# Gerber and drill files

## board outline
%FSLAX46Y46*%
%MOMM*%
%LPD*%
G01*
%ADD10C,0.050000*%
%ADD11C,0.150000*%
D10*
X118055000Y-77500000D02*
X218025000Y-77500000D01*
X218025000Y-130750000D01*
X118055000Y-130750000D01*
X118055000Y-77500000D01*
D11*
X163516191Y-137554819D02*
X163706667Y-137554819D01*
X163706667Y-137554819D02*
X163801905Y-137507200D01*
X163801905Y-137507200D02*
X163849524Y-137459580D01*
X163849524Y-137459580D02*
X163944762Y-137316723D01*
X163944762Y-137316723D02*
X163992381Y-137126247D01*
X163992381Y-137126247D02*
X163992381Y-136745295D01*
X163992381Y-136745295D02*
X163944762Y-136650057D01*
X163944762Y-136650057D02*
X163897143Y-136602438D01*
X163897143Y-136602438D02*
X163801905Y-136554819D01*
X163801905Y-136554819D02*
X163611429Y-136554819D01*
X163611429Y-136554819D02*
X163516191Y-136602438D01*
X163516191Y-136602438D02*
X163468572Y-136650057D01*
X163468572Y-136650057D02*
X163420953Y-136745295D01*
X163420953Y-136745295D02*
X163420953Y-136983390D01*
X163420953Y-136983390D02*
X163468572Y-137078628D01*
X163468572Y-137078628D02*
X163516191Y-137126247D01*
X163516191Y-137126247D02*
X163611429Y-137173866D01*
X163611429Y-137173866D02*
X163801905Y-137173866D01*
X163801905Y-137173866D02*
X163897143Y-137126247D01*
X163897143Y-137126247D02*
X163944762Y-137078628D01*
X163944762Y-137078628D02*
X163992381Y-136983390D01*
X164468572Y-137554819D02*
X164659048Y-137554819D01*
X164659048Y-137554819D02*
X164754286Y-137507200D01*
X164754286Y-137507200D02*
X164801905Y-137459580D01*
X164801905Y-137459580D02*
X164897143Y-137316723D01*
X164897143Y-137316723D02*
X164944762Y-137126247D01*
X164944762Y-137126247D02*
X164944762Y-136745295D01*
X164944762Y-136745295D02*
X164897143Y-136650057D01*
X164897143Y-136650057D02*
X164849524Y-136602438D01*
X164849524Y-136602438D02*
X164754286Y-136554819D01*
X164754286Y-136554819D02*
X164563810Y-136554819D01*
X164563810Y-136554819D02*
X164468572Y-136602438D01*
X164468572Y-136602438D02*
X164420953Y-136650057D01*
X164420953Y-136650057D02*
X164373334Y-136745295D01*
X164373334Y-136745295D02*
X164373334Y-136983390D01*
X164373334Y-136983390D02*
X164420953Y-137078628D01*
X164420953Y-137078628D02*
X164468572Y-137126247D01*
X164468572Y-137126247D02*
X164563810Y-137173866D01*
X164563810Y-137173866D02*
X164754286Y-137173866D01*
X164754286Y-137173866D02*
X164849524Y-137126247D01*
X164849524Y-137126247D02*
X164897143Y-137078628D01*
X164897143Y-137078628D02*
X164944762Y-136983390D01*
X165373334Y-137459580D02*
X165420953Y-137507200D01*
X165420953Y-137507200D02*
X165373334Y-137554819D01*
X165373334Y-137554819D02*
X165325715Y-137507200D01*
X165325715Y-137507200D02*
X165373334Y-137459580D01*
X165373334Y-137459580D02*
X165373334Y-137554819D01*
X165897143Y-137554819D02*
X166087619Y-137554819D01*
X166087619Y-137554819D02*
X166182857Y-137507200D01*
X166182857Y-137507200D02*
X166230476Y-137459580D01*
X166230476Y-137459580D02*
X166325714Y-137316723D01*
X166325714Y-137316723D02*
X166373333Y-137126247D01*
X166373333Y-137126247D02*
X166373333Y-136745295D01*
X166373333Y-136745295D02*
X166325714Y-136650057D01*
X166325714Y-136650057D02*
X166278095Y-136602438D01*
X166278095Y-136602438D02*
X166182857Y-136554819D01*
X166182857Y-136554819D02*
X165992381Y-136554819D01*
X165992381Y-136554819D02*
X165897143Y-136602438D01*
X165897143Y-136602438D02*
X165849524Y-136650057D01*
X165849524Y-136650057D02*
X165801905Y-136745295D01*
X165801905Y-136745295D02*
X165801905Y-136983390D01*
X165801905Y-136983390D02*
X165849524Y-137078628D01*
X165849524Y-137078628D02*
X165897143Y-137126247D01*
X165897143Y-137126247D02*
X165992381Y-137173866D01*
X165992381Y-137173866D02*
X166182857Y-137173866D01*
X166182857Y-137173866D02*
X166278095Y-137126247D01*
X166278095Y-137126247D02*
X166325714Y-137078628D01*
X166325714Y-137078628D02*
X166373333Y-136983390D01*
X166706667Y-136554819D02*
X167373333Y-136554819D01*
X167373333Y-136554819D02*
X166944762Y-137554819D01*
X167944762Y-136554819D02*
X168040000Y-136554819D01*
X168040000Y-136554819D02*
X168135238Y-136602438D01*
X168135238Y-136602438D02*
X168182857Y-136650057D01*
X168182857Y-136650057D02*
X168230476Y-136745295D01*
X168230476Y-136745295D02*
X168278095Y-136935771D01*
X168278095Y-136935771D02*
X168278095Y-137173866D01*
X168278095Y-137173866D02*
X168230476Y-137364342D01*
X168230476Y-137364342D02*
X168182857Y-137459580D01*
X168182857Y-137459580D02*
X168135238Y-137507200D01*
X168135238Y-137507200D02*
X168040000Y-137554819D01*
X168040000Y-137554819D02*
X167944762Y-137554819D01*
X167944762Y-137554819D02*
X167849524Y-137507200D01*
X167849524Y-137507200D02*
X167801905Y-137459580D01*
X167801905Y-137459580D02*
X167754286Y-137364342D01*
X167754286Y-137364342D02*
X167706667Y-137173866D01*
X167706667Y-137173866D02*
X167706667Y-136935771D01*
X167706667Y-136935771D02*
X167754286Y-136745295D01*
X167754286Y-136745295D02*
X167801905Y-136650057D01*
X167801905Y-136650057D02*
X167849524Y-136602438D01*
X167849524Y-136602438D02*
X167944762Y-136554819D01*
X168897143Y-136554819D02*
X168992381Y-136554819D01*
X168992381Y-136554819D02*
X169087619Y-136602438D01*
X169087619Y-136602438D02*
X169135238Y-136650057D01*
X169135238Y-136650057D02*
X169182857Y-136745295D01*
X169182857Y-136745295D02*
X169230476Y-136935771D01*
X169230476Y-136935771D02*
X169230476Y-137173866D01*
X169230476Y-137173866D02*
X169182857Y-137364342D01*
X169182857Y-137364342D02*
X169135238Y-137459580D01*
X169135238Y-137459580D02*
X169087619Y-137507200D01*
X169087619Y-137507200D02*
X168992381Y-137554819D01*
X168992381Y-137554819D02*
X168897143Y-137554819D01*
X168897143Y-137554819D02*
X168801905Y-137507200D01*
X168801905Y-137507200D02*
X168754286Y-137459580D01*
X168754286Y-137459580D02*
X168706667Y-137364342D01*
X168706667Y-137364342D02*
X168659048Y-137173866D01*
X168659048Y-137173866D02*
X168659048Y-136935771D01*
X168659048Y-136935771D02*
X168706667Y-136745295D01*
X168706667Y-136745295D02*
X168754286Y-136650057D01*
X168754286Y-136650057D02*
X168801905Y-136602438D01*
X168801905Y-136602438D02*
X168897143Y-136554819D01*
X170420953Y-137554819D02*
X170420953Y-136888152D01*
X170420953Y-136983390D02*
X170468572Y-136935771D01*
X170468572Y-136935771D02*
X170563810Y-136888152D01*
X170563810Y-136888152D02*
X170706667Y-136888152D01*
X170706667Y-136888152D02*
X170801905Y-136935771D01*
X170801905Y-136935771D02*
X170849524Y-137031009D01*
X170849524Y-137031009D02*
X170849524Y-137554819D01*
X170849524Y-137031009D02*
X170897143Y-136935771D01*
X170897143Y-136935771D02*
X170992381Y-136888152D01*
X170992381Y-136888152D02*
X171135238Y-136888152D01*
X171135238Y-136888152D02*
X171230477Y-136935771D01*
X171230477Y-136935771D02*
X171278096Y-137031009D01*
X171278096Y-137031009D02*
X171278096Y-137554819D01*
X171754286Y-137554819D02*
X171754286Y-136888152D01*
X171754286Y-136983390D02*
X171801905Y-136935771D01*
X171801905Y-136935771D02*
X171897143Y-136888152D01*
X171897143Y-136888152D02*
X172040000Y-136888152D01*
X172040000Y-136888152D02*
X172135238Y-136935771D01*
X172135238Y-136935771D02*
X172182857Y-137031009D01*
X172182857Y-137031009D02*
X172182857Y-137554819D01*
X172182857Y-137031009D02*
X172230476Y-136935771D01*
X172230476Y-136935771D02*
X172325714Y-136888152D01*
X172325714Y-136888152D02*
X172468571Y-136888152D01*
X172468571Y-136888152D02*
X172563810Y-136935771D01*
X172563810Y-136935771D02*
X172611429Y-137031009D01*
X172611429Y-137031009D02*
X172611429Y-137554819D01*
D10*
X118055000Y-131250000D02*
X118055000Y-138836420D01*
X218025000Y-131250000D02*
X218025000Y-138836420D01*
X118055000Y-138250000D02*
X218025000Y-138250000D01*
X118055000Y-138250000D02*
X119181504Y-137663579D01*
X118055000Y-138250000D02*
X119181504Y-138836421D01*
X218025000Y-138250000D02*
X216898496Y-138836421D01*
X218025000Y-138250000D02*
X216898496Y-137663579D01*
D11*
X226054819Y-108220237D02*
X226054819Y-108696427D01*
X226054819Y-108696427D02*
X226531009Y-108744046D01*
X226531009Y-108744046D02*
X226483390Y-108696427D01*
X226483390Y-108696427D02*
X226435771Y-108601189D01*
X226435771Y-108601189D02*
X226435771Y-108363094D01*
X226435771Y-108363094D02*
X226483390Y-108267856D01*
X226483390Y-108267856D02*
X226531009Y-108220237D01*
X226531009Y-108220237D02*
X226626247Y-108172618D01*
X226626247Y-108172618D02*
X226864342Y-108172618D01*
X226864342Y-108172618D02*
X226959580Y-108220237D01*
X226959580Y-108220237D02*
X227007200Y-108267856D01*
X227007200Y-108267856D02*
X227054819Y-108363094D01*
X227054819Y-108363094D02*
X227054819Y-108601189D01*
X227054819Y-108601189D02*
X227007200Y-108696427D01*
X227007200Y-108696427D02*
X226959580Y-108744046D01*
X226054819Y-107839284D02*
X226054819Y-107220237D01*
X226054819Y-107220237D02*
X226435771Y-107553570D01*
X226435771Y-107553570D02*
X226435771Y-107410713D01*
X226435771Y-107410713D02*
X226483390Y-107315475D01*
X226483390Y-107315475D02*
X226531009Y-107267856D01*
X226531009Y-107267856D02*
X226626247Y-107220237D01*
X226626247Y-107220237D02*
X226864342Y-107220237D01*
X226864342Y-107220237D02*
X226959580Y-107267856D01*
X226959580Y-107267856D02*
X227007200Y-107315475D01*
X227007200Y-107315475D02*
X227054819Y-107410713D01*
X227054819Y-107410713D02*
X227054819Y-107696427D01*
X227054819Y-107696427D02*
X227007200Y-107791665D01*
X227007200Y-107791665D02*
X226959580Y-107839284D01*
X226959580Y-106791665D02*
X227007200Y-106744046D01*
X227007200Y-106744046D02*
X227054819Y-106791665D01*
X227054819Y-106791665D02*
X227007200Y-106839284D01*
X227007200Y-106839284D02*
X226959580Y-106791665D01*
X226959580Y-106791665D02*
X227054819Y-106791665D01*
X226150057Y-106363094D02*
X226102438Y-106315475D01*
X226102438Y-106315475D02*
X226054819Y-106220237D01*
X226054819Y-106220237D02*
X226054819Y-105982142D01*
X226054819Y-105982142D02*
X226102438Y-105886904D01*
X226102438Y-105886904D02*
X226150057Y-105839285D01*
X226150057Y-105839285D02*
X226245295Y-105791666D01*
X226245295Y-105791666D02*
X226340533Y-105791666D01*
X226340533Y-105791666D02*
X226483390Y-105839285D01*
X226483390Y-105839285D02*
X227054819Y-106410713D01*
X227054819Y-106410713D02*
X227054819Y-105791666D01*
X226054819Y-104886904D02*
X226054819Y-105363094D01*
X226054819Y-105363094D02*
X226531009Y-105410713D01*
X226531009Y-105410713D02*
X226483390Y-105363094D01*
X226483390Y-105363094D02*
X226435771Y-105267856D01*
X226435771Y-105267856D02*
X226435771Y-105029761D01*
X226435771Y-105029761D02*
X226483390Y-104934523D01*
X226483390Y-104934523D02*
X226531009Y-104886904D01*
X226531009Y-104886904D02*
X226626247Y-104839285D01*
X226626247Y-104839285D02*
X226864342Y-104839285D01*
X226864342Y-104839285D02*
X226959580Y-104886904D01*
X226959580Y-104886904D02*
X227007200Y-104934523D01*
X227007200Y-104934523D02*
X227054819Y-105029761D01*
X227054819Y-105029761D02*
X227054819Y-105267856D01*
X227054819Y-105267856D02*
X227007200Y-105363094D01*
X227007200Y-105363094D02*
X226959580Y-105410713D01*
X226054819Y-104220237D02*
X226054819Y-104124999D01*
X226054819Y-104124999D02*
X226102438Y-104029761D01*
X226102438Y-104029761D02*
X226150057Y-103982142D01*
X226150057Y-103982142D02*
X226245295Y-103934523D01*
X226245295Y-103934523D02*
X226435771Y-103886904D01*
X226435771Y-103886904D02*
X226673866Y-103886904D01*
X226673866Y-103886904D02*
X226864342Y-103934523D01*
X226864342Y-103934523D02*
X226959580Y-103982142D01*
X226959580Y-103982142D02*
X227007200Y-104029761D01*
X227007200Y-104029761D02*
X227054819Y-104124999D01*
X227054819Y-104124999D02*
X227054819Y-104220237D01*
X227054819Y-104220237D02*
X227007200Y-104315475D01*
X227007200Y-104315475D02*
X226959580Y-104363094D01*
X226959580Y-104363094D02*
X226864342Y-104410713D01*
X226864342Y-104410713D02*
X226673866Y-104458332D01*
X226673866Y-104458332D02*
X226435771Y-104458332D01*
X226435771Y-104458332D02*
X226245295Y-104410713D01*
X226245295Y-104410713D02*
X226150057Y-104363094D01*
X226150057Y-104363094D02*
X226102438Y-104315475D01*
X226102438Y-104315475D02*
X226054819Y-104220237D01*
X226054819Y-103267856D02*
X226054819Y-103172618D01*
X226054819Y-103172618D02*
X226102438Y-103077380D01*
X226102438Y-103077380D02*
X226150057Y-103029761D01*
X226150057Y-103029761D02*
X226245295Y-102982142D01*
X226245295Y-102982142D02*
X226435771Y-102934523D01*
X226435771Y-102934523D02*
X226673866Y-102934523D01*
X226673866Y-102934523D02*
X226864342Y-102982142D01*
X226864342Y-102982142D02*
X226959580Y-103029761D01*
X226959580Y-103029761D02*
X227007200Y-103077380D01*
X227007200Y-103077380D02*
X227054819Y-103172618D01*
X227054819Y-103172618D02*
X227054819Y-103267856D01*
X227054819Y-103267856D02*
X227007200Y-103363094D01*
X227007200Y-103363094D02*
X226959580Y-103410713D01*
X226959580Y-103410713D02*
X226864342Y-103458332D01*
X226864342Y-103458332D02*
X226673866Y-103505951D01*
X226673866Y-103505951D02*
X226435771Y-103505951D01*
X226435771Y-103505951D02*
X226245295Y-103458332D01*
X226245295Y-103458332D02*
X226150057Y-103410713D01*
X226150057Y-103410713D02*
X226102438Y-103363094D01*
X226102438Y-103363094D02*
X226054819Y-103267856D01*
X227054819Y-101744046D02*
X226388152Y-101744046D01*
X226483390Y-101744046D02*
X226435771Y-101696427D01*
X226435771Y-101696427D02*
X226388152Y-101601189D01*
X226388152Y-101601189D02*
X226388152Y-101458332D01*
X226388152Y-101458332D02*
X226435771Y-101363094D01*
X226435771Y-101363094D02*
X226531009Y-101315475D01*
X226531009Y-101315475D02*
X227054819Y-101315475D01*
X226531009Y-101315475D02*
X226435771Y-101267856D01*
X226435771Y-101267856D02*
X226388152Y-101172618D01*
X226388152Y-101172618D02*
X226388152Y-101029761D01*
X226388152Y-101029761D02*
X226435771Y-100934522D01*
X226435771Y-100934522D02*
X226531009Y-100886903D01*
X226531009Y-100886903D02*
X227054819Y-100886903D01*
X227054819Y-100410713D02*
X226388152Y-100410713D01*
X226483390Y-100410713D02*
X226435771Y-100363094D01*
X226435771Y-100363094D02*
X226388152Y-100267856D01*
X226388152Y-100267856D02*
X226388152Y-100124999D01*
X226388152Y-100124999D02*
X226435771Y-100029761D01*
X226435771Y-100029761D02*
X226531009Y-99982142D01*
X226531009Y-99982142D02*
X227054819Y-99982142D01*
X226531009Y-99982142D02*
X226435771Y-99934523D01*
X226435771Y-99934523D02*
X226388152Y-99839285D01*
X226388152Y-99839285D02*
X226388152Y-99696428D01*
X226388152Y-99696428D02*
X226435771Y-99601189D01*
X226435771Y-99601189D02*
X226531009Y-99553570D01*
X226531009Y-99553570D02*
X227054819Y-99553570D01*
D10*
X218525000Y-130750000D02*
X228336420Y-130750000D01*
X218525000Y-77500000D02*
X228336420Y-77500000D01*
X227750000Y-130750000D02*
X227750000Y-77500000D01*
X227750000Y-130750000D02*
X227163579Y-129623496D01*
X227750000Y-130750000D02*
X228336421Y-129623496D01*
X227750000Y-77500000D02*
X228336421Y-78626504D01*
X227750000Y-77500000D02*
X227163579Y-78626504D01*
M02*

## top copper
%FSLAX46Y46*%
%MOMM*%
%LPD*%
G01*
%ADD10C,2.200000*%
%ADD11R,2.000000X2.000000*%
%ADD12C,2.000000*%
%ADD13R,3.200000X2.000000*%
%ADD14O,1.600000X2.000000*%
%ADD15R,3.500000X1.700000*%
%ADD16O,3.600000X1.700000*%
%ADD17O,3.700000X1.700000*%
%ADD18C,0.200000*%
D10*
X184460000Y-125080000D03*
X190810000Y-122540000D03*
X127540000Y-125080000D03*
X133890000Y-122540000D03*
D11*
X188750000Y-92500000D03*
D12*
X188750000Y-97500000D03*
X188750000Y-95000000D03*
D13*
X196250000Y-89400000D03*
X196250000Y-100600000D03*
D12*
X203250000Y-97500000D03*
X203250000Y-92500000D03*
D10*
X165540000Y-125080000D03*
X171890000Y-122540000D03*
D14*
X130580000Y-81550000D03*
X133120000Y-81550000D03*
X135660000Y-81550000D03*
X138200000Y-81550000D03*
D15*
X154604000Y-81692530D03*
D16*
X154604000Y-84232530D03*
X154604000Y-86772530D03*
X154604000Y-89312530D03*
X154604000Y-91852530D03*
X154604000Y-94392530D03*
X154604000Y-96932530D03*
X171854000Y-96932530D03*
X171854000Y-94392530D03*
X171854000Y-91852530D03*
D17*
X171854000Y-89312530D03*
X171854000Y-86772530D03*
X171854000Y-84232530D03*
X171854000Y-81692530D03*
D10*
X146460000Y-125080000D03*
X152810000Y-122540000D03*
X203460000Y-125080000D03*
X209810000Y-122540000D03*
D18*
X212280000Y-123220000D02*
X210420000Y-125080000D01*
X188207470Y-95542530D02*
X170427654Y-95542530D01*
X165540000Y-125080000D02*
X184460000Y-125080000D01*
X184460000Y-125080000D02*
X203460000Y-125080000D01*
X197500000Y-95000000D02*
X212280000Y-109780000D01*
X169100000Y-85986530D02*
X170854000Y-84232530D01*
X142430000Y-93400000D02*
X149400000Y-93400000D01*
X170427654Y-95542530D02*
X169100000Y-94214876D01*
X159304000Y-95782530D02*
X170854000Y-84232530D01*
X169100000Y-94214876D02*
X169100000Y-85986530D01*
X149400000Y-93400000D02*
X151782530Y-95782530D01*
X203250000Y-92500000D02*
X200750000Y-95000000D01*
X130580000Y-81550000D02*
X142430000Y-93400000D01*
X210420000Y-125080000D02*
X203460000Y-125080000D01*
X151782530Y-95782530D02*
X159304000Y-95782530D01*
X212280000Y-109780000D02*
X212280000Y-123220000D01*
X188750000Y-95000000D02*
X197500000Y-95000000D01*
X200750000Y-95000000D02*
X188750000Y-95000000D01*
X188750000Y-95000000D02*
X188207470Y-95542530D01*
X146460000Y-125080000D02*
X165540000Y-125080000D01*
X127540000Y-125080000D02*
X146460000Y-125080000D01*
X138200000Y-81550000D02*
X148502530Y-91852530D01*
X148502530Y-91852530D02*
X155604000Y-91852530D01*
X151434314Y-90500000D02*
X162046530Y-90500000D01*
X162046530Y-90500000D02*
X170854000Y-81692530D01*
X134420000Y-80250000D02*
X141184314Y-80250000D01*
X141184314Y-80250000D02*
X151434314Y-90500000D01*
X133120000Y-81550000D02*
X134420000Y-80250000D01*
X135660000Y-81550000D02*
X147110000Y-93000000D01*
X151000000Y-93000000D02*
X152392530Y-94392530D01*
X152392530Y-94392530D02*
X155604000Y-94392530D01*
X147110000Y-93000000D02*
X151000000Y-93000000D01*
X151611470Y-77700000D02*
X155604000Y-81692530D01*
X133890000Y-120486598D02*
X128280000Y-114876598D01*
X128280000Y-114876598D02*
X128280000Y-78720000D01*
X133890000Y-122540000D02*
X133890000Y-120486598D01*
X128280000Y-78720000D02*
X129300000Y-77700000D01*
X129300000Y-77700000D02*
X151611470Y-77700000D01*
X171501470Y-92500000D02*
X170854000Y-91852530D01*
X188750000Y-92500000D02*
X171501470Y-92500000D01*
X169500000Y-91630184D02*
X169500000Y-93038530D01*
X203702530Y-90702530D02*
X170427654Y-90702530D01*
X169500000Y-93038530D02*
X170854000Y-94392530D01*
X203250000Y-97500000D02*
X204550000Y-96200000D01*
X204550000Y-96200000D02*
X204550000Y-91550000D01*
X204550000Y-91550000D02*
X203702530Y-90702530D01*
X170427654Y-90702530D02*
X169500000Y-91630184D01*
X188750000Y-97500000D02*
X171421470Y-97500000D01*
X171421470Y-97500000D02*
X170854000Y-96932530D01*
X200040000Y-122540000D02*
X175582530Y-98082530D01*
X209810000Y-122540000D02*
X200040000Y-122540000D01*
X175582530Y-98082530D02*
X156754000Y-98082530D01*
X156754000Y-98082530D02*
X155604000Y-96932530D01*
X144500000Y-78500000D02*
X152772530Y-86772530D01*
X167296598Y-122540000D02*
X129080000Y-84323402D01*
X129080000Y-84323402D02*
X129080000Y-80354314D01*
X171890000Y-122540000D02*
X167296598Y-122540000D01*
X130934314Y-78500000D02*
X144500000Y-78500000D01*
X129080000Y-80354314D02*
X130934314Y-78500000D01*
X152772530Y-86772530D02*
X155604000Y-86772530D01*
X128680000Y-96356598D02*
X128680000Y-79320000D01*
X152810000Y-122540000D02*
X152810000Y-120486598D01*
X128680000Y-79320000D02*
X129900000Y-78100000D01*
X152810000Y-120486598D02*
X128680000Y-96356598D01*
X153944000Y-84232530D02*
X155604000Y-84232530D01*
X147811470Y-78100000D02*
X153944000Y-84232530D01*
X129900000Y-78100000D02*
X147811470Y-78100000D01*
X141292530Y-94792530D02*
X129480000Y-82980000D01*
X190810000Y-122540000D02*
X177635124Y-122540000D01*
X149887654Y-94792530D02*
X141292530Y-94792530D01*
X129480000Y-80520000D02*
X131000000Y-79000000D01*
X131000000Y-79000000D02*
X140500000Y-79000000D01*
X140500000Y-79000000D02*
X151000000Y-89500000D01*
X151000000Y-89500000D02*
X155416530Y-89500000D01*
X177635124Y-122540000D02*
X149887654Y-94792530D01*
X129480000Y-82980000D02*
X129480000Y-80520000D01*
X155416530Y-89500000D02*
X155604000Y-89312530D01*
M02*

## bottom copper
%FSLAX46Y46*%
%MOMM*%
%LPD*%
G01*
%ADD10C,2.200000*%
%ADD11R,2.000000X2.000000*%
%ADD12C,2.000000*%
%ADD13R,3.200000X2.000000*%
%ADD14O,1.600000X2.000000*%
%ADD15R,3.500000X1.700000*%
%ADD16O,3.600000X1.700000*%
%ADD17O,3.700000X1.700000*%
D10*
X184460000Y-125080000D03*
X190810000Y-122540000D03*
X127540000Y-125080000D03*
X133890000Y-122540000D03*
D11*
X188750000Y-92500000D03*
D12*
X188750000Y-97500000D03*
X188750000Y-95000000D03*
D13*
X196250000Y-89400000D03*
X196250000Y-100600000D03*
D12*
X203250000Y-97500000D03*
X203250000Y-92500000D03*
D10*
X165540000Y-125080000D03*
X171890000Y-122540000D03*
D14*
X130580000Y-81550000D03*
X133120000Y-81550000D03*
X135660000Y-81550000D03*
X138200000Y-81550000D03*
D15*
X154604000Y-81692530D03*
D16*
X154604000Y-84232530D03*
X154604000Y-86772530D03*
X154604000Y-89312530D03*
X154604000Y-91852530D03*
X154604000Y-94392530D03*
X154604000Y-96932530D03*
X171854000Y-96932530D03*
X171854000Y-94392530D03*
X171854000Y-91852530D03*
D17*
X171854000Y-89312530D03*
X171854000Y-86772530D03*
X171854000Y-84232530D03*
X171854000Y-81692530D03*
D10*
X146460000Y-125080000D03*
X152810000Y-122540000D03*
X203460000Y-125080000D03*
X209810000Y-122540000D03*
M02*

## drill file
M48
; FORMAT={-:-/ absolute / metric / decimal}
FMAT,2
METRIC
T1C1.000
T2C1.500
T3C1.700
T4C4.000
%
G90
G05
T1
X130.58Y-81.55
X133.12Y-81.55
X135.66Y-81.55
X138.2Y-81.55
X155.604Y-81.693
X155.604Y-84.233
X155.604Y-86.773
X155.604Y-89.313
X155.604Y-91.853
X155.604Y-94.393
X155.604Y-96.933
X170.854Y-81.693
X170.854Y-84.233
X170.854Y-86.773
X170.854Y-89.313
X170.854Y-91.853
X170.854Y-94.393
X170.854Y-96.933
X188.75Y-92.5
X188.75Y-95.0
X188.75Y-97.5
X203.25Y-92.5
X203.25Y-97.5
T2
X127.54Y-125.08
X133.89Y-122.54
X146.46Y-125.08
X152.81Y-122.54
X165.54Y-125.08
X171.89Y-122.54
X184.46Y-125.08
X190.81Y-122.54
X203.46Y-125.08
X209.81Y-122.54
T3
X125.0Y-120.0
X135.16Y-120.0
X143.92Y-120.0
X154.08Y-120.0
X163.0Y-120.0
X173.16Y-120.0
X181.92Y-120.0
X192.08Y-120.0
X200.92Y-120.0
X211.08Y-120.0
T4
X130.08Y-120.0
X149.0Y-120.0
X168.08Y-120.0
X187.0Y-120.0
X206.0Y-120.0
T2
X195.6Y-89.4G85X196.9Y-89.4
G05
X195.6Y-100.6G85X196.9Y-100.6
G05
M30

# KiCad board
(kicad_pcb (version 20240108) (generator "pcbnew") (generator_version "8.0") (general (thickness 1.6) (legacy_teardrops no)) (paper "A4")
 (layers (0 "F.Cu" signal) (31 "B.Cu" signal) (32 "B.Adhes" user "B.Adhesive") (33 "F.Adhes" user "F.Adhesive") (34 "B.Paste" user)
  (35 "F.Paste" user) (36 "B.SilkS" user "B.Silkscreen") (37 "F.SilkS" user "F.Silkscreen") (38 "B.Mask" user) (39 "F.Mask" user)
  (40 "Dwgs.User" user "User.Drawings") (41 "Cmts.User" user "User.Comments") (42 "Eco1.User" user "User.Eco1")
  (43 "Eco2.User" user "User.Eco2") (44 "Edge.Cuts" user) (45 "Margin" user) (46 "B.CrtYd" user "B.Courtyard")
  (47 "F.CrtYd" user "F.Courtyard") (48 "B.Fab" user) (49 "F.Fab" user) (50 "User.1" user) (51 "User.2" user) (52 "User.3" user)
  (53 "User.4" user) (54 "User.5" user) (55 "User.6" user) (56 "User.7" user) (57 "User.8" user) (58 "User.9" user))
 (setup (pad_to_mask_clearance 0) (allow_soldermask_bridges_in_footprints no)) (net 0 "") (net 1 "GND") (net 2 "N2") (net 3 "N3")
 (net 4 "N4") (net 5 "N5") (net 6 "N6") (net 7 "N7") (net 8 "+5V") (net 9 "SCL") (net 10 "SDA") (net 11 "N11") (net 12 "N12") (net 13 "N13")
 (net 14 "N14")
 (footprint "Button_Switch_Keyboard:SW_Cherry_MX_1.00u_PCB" (layer "F.Cu") (at 184.46 125.08 180)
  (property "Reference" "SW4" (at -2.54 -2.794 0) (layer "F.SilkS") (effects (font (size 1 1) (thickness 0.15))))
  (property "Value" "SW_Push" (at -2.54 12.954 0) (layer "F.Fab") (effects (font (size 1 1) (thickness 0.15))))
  (pad "" np_thru_hole circle (at -7.62 5.08 180) (size 1.7 1.7) (drill 1.7) (layers "*.Cu" "*.Mask"))
  (pad "" np_thru_hole circle (at -2.54 5.08 180) (size 4 4) (drill 4) (layers "*.Cu" "*.Mask"))
  (pad "" np_thru_hole circle (at 2.54 5.08 180) (size 1.7 1.7) (drill 1.7) (layers "*.Cu" "*.Mask"))
  (pad "1" thru_hole circle (at 0 0 180) (size 2.2 2.2) (drill 1.5) (layers "*.Cu" "*.Mask") (remove_unused_layers no) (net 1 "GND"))
  (pad "2" thru_hole circle (at -6.35 2.54 180) (size 2.2 2.2) (drill 1.5) (layers "*.Cu" "*.Mask") (remove_unused_layers no) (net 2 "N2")))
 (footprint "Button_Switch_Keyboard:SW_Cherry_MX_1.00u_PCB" (layer "F.Cu") (at 127.54 125.08 180)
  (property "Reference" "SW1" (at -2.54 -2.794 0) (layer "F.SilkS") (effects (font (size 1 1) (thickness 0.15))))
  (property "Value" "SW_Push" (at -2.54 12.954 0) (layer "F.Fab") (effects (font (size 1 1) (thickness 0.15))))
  (pad "" np_thru_hole circle (at -7.62 5.08 180) (size 1.7 1.7) (drill 1.7) (layers "*.Cu" "*.Mask"))
  (pad "" np_thru_hole circle (at -2.54 5.08 180) (size 4 4) (drill 4) (layers "*.Cu" "*.Mask"))
  (pad "" np_thru_hole circle (at 2.54 5.08 180) (size 1.7 1.7) (drill 1.7) (layers "*.Cu" "*.Mask"))
  (pad "1" thru_hole circle (at 0 0 180) (size 2.2 2.2) (drill 1.5) (layers "*.Cu" "*.Mask") (remove_unused_layers no) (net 1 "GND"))
  (pad "2" thru_hole circle (at -6.35 2.54 180) (size 2.2 2.2) (drill 1.5) (layers "*.Cu" "*.Mask") (remove_unused_layers no) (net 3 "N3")))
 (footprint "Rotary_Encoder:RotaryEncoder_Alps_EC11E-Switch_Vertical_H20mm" (layer "F.Cu") (at 188.75 92.5)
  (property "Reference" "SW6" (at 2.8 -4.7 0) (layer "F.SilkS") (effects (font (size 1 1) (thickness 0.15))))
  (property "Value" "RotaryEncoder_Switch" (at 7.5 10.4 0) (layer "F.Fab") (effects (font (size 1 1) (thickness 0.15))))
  (pad "A" thru_hole rect (at 0 0) (size 2 2) (drill 1) (layers "*.Cu" "*.Mask") (remove_unused_layers no) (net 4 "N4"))
  (pad "B" thru_hole circle (at 0 5) (size 2 2) (drill 1) (layers "*.Cu" "*.Mask") (remove_unused_layers no) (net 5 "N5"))
  (pad "C" thru_hole circle (at 0 2.5) (size 2 2) (drill 1) (layers "*.Cu" "*.Mask") (remove_unused_layers no) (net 1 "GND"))
  (pad "MP" thru_hole rect (at 7.5 -3.1) (size 3.2 2) (drill oval 2.8 1.5) (layers "*.Cu" "*.Mask") (remove_unused_layers no))
  (pad "MP" thru_hole rect (at 7.5 8.1) (size 3.2 2) (drill oval 2.8 1.5) (layers "*.Cu" "*.Mask") (remove_unused_layers no))
  (pad "S1" thru_hole circle (at 14.5 5) (size 2 2) (drill 1) (layers "*.Cu" "*.Mask") (remove_unused_layers no) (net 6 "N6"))
  (pad "S2" thru_hole circle (at 14.5 0) (size 2 2) (drill 1) (layers "*.Cu" "*.Mask") (remove_unused_layers no) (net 1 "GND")))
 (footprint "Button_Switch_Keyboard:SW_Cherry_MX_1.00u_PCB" (layer "F.Cu") (at 165.54 125.08 180)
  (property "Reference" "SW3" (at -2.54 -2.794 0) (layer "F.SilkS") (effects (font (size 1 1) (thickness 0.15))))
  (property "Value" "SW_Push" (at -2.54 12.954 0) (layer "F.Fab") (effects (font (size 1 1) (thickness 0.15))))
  (pad "" np_thru_hole circle (at -7.62 5.08 180) (size 1.7 1.7) (drill 1.7) (layers "*.Cu" "*.Mask"))
  (pad "" np_thru_hole circle (at -2.54 5.08 180) (size 4 4) (drill 4) (layers "*.Cu" "*.Mask"))
  (pad "" np_thru_hole circle (at 2.54 5.08 180) (size 1.7 1.7) (drill 1.7) (layers "*.Cu" "*.Mask"))
  (pad "1" thru_hole circle (at 0 0 180) (size 2.2 2.2) (drill 1.5) (layers "*.Cu" "*.Mask") (remove_unused_layers no) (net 1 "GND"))
  (pad "2" thru_hole circle (at -6.35 2.54 180) (size 2.2 2.2) (drill 1.5) (layers "*.Cu" "*.Mask") (remove_unused_layers no) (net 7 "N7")))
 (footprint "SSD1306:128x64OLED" (layer "F.Cu") (at 134.2 92.15)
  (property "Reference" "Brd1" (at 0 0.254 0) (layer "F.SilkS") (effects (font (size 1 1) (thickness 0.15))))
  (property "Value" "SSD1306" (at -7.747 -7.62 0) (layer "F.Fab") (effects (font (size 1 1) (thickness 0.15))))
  (pad "1" thru_hole oval (at -3.62 -10.6 90) (size 2 1.6) (drill 1) (layers "*.Cu" "*.Mask") (remove_unused_layers no) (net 1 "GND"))
  (pad "2" thru_hole oval (at -1.08 -10.6 90) (size 2 1.6) (drill 1) (layers "*.Cu" "*.Mask") (remove_unused_layers no) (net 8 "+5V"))
  (pad "3" thru_hole oval (at 1.46 -10.6 90) (size 2 1.6) (drill 1) (layers "*.Cu" "*.Mask") (remove_unused_layers no) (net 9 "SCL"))
  (pad "4" thru_hole oval (at 4 -10.6 90) (size 2 1.6) (drill 1) (layers "*.Cu" "*.Mask") (remove_unused_layers no) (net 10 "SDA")))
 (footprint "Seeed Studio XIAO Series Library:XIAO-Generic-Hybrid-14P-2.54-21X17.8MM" (layer "F.Cu") (at 163.229 89.31253)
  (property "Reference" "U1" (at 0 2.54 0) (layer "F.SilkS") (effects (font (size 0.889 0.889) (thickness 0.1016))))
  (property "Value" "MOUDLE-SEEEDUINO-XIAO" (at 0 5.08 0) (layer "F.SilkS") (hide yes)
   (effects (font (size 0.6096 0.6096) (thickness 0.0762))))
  (pad "1" thru_hole rect (at -7.625 -7.62) (size 3.5 1.7) (drill 1 (offset -1 0)) (layers "*.Cu" "*.Mask") (remove_unused_layers no)
   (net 3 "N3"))
  (pad "2" thru_hole oval (at -7.625 -5.08) (size 3.6 1.7) (drill 1 (offset -1 0)) (layers "*.Cu" "*.Mask") (remove_unused_layers no)
   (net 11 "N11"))
  (pad "3" thru_hole oval (at -7.625 -2.54) (size 3.6 1.7) (drill 1 (offset -1 0)) (layers "*.Cu" "*.Mask") (remove_unused_layers no)
   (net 7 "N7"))
  (pad "4" thru_hole oval (at -7.625 0) (size 3.6 1.7) (drill 1 (offset -1 0)) (layers "*.Cu" "*.Mask") (remove_unused_layers no)
   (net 2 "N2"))
  (pad "5" thru_hole oval (at -7.625 2.54) (size 3.6 1.7) (drill 1 (offset -1 0)) (layers "*.Cu" "*.Mask") (remove_unused_layers no)
   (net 10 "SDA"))
  (pad "6" thru_hole oval (at -7.625 5.08 180) (size 3.6 1.7) (drill 1 (offset 1 0)) (layers "*.Cu" "*.Mask") (remove_unused_layers no)
   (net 9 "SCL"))
  (pad "7" thru_hole oval (at -7.625 7.62) (size 3.6 1.7) (drill 1 (offset -1 0)) (layers "*.Cu" "*.Mask") (remove_unused_layers no)
   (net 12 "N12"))
  (pad "8" thru_hole oval (at 7.625 7.62) (size 3.6 1.7) (drill 1 (offset 1 0)) (layers "*.Cu" "*.Mask") (remove_unused_layers no)
   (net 5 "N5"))
  (pad "9" thru_hole oval (at 7.625 5.08) (size 3.6 1.7) (drill 1 (offset 1 0)) (layers "*.Cu" "*.Mask") (remove_unused_layers no)
   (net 6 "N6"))
  (pad "10" thru_hole oval (at 7.625 2.54) (size 3.6 1.7) (drill 1 (offset 1 0)) (layers "*.Cu" "*.Mask") (remove_unused_layers no)
   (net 4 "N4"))
  (pad "11" thru_hole oval (at 7.625 0) (size 3.7 1.7) (drill 1 (offset 1 0)) (layers "*.Cu" "*.Mask") (remove_unused_layers no)
   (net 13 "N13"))
  (pad "12" thru_hole oval (at 7.625 -2.54) (size 3.7 1.7) (drill 1 (offset 1 0)) (layers "*.Cu" "*.Mask") (remove_unused_layers no)
   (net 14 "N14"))
  (pad "13" thru_hole oval (at 7.625 -5.08) (size 3.7 1.7) (drill 1 (offset 1 0)) (layers "*.Cu" "*.Mask") (remove_unused_layers no)
   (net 1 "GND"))
  (pad "14" thru_hole oval (at 7.625 -7.62) (size 3.7 1.7) (drill 1 (offset 1 0)) (layers "*.Cu" "*.Mask") (remove_unused_layers no)
   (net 8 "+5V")))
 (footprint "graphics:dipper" (layer "F.Cu") (at 183.488038 81.796655 90)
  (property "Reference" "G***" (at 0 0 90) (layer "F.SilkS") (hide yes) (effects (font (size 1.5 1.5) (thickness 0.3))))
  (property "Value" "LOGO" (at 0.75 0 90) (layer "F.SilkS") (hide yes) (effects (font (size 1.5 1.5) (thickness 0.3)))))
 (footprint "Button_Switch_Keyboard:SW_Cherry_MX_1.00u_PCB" (layer "F.Cu") (at 146.46 125.08 180)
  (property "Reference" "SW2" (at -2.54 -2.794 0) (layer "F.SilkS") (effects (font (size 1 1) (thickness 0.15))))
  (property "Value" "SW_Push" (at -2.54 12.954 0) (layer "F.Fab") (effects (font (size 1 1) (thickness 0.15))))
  (pad "" np_thru_hole circle (at -7.62 5.08 180) (size 1.7 1.7) (drill 1.7) (layers "*.Cu" "*.Mask"))
  (pad "" np_thru_hole circle (at -2.54 5.08 180) (size 4 4) (drill 4) (layers "*.Cu" "*.Mask"))
  (pad "" np_thru_hole circle (at 2.54 5.08 180) (size 1.7 1.7) (drill 1.7) (layers "*.Cu" "*.Mask"))
  (pad "1" thru_hole circle (at 0 0 180) (size 2.2 2.2) (drill 1.5) (layers "*.Cu" "*.Mask") (remove_unused_layers no) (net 1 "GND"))
  (pad "2" thru_hole circle (at -6.35 2.54 180) (size 2.2 2.2) (drill 1.5) (layers "*.Cu" "*.Mask") (remove_unused_layers no) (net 11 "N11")))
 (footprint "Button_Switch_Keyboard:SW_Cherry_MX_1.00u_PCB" (layer "F.Cu") (at 203.46 125.08 180)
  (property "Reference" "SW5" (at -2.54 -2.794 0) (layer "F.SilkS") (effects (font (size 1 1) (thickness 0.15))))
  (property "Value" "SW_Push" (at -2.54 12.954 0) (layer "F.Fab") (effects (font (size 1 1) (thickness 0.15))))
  (pad "" np_thru_hole circle (at -7.62 5.08 180) (size 1.7 1.7) (drill 1.7) (layers "*.Cu" "*.Mask"))
  (pad "" np_thru_hole circle (at -2.54 5.08 180) (size 4 4) (drill 4) (layers "*.Cu" "*.Mask"))
  (pad "" np_thru_hole circle (at 2.54 5.08 180) (size 1.7 1.7) (drill 1.7) (layers "*.Cu" "*.Mask"))
  (pad "1" thru_hole circle (at 0 0 180) (size 2.2 2.2) (drill 1.5) (layers "*.Cu" "*.Mask") (remove_unused_layers no) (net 1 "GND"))
  (pad "2" thru_hole circle (at -6.35 2.54 180) (size 2.2 2.2) (drill 1.5) (layers "*.Cu" "*.Mask") (remove_unused_layers no) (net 12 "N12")))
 (gr_rect (start 118.055 77.5) (end 218.025 130.75) (stroke (width 0.05) (type default)) (fill none) (layer "Edge.Cuts"))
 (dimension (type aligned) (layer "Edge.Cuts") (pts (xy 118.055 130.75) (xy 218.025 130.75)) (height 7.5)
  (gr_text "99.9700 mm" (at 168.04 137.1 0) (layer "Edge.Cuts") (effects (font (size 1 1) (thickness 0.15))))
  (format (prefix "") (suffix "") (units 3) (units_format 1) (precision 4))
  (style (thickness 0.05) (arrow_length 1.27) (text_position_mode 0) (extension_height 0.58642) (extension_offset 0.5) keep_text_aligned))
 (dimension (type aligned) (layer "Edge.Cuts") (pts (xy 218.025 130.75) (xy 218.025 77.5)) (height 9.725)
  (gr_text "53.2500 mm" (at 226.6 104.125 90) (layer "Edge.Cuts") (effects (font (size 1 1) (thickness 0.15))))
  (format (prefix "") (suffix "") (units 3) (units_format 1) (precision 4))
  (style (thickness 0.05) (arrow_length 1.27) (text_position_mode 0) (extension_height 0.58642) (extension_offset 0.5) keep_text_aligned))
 (segment (start 212.28 123.22) (end 210.42 125.08) (width 0.2) (layer "F.Cu") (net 1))
 (segment (start 188.20747 95.54253) (end 170.427654 95.54253) (width 0.2) (layer "F.Cu") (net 1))
 (segment (start 165.54 125.08) (end 184.46 125.08) (width 0.2) (layer "F.Cu") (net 1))
 (segment (start 184.46 125.08) (end 203.46 125.08) (width 0.2) (layer "F.Cu") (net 1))
 (segment (start 197.5 95) (end 212.28 109.78) (width 0.2) (layer "F.Cu") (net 1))
 (segment (start 169.1 85.98653) (end 170.854 84.23253) (width 0.2) (layer "F.Cu") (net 1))
 (segment (start 142.43 93.4) (end 149.4 93.4) (width 0.2) (layer "F.Cu") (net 1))
 (segment (start 170.427654 95.54253) (end 169.1 94.214876) (width 0.2) (layer "F.Cu") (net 1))
 (segment (start 159.304 95.78253) (end 170.854 84.23253) (width 0.2) (layer "F.Cu") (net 1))
 (segment (start 169.1 94.214876) (end 169.1 85.98653) (width 0.2) (layer "F.Cu") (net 1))
 (segment (start 149.4 93.4) (end 151.78253 95.78253) (width 0.2) (layer "F.Cu") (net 1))
 (segment (start 203.25 92.5) (end 200.75 95) (width 0.2) (layer "F.Cu") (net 1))
 (segment (start 130.58 81.55) (end 142.43 93.4) (width 0.2) (layer "F.Cu") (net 1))
 (segment (start 210.42 125.08) (end 203.46 125.08) (width 0.2) (layer "F.Cu") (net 1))
 (segment (start 151.78253 95.78253) (end 159.304 95.78253) (width 0.2) (layer "F.Cu") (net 1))
 (segment (start 212.28 109.78) (end 212.28 123.22) (width 0.2) (layer "F.Cu") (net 1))
 (segment (start 188.75 95) (end 197.5 95) (width 0.2) (layer "F.Cu") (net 1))
 (segment (start 200.75 95) (end 188.75 95) (width 0.2) (layer "F.Cu") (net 1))
 (segment (start 188.75 95) (end 188.20747 95.54253) (width 0.2) (layer "F.Cu") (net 1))
 (segment (start 146.46 125.08) (end 165.54 125.08) (width 0.2) (layer "F.Cu") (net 1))
 (segment (start 127.54 125.08) (end 146.46 125.08) (width 0.2) (layer "F.Cu") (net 1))
 (segment (start 138.2 81.55) (end 148.50253 91.85253) (width 0.2) (layer "F.Cu") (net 10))
 (segment (start 148.50253 91.85253) (end 155.604 91.85253) (width 0.2) (layer "F.Cu") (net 10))
 (segment (start 151.434314 90.5) (end 162.04653 90.5) (width 0.2) (layer "F.Cu") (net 8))
 (segment (start 162.04653 90.5) (end 170.854 81.69253) (width 0.2) (layer "F.Cu") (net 8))
 (segment (start 134.42 80.25) (end 141.184314 80.25) (width 0.2) (layer "F.Cu") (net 8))
 (segment (start 141.184314 80.25) (end 151.434314 90.5) (width 0.2) (layer "F.Cu") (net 8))
 (segment (start 133.12 81.55) (end 134.42 80.25) (width 0.2) (layer "F.Cu") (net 8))
 (segment (start 135.66 81.55) (end 147.11 93) (width 0.2) (layer "F.Cu") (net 9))
 (segment (start 151 93) (end 152.39253 94.39253) (width 0.2) (layer "F.Cu") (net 9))
 (segment (start 152.39253 94.39253) (end 155.604 94.39253) (width 0.2) (layer "F.Cu") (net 9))
 (segment (start 147.11 93) (end 151 93) (width 0.2) (layer "F.Cu") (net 9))
 (segment (start 151.61147 77.7) (end 155.604 81.69253) (width 0.2) (layer "F.Cu") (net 3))
 (segment (start 133.89 120.486598) (end 128.28 114.876598) (width 0.2) (layer "F.Cu") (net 3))
 (segment (start 128.28 114.876598) (end 128.28 78.72) (width 0.2) (layer "F.Cu") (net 3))
 (segment (start 133.89 122.54) (end 133.89 120.486598) (width 0.2) (layer "F.Cu") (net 3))
 (segment (start 128.28 78.72) (end 129.3 77.7) (width 0.2) (layer "F.Cu") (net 3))
 (segment (start 129.3 77.7) (end 151.61147 77.7) (width 0.2) (layer "F.Cu") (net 3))
 (segment (start 171.50147 92.5) (end 170.854 91.85253) (width 0.2) (layer "F.Cu") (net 4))
 (segment (start 188.75 92.5) (end 171.50147 92.5) (width 0.2) (layer "F.Cu") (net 4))
 (segment (start 169.5 91.630184) (end 169.5 93.03853) (width 0.2) (layer "F.Cu") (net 6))
 (segment (start 203.70253 90.70253) (end 170.427654 90.70253) (width 0.2) (layer "F.Cu") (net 6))
 (segment (start 169.5 93.03853) (end 170.854 94.39253) (width 0.2) (layer "F.Cu") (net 6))
 (segment (start 203.25 97.5) (end 204.55 96.2) (width 0.2) (layer "F.Cu") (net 6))
 (segment (start 204.55 96.2) (end 204.55 91.55) (width 0.2) (layer "F.Cu") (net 6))
 (segment (start 204.55 91.55) (end 203.70253 90.70253) (width 0.2) (layer "F.Cu") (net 6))
 (segment (start 170.427654 90.70253) (end 169.5 91.630184) (width 0.2) (layer "F.Cu") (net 6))
 (segment (start 188.75 97.5) (end 171.42147 97.5) (width 0.2) (layer "F.Cu") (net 5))
 (segment (start 171.42147 97.5) (end 170.854 96.93253) (width 0.2) (layer "F.Cu") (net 5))
 (segment (start 200.04 122.54) (end 175.58253 98.08253) (width 0.2) (layer "F.Cu") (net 12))
 (segment (start 209.81 122.54) (end 200.04 122.54) (width 0.2) (layer "F.Cu") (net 12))
 (segment (start 175.58253 98.08253) (end 156.754 98.08253) (width 0.2) (layer "F.Cu") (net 12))
 (segment (start 156.754 98.08253) (end 155.604 96.93253) (width 0.2) (layer "F.Cu") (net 12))
 (segment (start 144.5 78.5) (end 152.77253 86.77253) (width 0.2) (layer "F.Cu") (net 7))
 (segment (start 167.296598 122.54) (end 129.08 84.323402) (width 0.2) (layer "F.Cu") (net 7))
 (segment (start 129.08 84.323402) (end 129.08 80.354314) (width 0.2) (layer "F.Cu") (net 7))
 (segment (start 171.89 122.54) (end 167.296598 122.54) (width 0.2) (layer "F.Cu") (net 7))
 (segment (start 130.934314 78.5) (end 144.5 78.5) (width 0.2) (layer "F.Cu") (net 7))
 (segment (start 129.08 80.354314) (end 130.934314 78.5) (width 0.2) (layer "F.Cu") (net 7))
 (segment (start 152.77253 86.77253) (end 155.604 86.77253) (width 0.2) (layer "F.Cu") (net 7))
 (segment (start 128.68 96.356598) (end 128.68 79.32) (width 0.2) (layer "F.Cu") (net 11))
 (segment (start 152.81 122.54) (end 152.81 120.486598) (width 0.2) (layer "F.Cu") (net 11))
 (segment (start 128.68 79.32) (end 129.9 78.1) (width 0.2) (layer "F.Cu") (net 11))
 (segment (start 152.81 120.486598) (end 128.68 96.356598) (width 0.2) (layer "F.Cu") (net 11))
 (segment (start 153.944 84.23253) (end 155.604 84.23253) (width 0.2) (layer "F.Cu") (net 11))
 (segment (start 147.81147 78.1) (end 153.944 84.23253) (width 0.2) (layer "F.Cu") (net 11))
 (segment (start 129.9 78.1) (end 147.81147 78.1) (width 0.2) (layer "F.Cu") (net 11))
 (segment (start 141.29253 94.79253) (end 129.48 82.98) (width 0.2) (layer "F.Cu") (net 2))
 (segment (start 190.81 122.54) (end 177.635124 122.54) (width 0.2) (layer "F.Cu") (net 2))
 (segment (start 149.887654 94.79253) (end 141.29253 94.79253) (width 0.2) (layer "F.Cu") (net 2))
 (segment (start 129.48 80.52) (end 131 79) (width 0.2) (layer "F.Cu") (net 2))
 (segment (start 131 79) (end 140.5 79) (width 0.2) (layer "F.Cu") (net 2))
 (segment (start 140.5 79) (end 151 89.5) (width 0.2) (layer "F.Cu") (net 2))
 (segment (start 151 89.5) (end 155.41653 89.5) (width 0.2) (layer "F.Cu") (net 2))
 (segment (start 177.635124 122.54) (end 149.887654 94.79253) (width 0.2) (layer "F.Cu") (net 2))
 (segment (start 129.48 82.98) (end 129.48 80.52) (width 0.2) (layer "F.Cu") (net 2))
 (segment (start 155.41653 89.5) (end 155.604 89.31253) (width 0.2) (layer "F.Cu") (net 2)))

